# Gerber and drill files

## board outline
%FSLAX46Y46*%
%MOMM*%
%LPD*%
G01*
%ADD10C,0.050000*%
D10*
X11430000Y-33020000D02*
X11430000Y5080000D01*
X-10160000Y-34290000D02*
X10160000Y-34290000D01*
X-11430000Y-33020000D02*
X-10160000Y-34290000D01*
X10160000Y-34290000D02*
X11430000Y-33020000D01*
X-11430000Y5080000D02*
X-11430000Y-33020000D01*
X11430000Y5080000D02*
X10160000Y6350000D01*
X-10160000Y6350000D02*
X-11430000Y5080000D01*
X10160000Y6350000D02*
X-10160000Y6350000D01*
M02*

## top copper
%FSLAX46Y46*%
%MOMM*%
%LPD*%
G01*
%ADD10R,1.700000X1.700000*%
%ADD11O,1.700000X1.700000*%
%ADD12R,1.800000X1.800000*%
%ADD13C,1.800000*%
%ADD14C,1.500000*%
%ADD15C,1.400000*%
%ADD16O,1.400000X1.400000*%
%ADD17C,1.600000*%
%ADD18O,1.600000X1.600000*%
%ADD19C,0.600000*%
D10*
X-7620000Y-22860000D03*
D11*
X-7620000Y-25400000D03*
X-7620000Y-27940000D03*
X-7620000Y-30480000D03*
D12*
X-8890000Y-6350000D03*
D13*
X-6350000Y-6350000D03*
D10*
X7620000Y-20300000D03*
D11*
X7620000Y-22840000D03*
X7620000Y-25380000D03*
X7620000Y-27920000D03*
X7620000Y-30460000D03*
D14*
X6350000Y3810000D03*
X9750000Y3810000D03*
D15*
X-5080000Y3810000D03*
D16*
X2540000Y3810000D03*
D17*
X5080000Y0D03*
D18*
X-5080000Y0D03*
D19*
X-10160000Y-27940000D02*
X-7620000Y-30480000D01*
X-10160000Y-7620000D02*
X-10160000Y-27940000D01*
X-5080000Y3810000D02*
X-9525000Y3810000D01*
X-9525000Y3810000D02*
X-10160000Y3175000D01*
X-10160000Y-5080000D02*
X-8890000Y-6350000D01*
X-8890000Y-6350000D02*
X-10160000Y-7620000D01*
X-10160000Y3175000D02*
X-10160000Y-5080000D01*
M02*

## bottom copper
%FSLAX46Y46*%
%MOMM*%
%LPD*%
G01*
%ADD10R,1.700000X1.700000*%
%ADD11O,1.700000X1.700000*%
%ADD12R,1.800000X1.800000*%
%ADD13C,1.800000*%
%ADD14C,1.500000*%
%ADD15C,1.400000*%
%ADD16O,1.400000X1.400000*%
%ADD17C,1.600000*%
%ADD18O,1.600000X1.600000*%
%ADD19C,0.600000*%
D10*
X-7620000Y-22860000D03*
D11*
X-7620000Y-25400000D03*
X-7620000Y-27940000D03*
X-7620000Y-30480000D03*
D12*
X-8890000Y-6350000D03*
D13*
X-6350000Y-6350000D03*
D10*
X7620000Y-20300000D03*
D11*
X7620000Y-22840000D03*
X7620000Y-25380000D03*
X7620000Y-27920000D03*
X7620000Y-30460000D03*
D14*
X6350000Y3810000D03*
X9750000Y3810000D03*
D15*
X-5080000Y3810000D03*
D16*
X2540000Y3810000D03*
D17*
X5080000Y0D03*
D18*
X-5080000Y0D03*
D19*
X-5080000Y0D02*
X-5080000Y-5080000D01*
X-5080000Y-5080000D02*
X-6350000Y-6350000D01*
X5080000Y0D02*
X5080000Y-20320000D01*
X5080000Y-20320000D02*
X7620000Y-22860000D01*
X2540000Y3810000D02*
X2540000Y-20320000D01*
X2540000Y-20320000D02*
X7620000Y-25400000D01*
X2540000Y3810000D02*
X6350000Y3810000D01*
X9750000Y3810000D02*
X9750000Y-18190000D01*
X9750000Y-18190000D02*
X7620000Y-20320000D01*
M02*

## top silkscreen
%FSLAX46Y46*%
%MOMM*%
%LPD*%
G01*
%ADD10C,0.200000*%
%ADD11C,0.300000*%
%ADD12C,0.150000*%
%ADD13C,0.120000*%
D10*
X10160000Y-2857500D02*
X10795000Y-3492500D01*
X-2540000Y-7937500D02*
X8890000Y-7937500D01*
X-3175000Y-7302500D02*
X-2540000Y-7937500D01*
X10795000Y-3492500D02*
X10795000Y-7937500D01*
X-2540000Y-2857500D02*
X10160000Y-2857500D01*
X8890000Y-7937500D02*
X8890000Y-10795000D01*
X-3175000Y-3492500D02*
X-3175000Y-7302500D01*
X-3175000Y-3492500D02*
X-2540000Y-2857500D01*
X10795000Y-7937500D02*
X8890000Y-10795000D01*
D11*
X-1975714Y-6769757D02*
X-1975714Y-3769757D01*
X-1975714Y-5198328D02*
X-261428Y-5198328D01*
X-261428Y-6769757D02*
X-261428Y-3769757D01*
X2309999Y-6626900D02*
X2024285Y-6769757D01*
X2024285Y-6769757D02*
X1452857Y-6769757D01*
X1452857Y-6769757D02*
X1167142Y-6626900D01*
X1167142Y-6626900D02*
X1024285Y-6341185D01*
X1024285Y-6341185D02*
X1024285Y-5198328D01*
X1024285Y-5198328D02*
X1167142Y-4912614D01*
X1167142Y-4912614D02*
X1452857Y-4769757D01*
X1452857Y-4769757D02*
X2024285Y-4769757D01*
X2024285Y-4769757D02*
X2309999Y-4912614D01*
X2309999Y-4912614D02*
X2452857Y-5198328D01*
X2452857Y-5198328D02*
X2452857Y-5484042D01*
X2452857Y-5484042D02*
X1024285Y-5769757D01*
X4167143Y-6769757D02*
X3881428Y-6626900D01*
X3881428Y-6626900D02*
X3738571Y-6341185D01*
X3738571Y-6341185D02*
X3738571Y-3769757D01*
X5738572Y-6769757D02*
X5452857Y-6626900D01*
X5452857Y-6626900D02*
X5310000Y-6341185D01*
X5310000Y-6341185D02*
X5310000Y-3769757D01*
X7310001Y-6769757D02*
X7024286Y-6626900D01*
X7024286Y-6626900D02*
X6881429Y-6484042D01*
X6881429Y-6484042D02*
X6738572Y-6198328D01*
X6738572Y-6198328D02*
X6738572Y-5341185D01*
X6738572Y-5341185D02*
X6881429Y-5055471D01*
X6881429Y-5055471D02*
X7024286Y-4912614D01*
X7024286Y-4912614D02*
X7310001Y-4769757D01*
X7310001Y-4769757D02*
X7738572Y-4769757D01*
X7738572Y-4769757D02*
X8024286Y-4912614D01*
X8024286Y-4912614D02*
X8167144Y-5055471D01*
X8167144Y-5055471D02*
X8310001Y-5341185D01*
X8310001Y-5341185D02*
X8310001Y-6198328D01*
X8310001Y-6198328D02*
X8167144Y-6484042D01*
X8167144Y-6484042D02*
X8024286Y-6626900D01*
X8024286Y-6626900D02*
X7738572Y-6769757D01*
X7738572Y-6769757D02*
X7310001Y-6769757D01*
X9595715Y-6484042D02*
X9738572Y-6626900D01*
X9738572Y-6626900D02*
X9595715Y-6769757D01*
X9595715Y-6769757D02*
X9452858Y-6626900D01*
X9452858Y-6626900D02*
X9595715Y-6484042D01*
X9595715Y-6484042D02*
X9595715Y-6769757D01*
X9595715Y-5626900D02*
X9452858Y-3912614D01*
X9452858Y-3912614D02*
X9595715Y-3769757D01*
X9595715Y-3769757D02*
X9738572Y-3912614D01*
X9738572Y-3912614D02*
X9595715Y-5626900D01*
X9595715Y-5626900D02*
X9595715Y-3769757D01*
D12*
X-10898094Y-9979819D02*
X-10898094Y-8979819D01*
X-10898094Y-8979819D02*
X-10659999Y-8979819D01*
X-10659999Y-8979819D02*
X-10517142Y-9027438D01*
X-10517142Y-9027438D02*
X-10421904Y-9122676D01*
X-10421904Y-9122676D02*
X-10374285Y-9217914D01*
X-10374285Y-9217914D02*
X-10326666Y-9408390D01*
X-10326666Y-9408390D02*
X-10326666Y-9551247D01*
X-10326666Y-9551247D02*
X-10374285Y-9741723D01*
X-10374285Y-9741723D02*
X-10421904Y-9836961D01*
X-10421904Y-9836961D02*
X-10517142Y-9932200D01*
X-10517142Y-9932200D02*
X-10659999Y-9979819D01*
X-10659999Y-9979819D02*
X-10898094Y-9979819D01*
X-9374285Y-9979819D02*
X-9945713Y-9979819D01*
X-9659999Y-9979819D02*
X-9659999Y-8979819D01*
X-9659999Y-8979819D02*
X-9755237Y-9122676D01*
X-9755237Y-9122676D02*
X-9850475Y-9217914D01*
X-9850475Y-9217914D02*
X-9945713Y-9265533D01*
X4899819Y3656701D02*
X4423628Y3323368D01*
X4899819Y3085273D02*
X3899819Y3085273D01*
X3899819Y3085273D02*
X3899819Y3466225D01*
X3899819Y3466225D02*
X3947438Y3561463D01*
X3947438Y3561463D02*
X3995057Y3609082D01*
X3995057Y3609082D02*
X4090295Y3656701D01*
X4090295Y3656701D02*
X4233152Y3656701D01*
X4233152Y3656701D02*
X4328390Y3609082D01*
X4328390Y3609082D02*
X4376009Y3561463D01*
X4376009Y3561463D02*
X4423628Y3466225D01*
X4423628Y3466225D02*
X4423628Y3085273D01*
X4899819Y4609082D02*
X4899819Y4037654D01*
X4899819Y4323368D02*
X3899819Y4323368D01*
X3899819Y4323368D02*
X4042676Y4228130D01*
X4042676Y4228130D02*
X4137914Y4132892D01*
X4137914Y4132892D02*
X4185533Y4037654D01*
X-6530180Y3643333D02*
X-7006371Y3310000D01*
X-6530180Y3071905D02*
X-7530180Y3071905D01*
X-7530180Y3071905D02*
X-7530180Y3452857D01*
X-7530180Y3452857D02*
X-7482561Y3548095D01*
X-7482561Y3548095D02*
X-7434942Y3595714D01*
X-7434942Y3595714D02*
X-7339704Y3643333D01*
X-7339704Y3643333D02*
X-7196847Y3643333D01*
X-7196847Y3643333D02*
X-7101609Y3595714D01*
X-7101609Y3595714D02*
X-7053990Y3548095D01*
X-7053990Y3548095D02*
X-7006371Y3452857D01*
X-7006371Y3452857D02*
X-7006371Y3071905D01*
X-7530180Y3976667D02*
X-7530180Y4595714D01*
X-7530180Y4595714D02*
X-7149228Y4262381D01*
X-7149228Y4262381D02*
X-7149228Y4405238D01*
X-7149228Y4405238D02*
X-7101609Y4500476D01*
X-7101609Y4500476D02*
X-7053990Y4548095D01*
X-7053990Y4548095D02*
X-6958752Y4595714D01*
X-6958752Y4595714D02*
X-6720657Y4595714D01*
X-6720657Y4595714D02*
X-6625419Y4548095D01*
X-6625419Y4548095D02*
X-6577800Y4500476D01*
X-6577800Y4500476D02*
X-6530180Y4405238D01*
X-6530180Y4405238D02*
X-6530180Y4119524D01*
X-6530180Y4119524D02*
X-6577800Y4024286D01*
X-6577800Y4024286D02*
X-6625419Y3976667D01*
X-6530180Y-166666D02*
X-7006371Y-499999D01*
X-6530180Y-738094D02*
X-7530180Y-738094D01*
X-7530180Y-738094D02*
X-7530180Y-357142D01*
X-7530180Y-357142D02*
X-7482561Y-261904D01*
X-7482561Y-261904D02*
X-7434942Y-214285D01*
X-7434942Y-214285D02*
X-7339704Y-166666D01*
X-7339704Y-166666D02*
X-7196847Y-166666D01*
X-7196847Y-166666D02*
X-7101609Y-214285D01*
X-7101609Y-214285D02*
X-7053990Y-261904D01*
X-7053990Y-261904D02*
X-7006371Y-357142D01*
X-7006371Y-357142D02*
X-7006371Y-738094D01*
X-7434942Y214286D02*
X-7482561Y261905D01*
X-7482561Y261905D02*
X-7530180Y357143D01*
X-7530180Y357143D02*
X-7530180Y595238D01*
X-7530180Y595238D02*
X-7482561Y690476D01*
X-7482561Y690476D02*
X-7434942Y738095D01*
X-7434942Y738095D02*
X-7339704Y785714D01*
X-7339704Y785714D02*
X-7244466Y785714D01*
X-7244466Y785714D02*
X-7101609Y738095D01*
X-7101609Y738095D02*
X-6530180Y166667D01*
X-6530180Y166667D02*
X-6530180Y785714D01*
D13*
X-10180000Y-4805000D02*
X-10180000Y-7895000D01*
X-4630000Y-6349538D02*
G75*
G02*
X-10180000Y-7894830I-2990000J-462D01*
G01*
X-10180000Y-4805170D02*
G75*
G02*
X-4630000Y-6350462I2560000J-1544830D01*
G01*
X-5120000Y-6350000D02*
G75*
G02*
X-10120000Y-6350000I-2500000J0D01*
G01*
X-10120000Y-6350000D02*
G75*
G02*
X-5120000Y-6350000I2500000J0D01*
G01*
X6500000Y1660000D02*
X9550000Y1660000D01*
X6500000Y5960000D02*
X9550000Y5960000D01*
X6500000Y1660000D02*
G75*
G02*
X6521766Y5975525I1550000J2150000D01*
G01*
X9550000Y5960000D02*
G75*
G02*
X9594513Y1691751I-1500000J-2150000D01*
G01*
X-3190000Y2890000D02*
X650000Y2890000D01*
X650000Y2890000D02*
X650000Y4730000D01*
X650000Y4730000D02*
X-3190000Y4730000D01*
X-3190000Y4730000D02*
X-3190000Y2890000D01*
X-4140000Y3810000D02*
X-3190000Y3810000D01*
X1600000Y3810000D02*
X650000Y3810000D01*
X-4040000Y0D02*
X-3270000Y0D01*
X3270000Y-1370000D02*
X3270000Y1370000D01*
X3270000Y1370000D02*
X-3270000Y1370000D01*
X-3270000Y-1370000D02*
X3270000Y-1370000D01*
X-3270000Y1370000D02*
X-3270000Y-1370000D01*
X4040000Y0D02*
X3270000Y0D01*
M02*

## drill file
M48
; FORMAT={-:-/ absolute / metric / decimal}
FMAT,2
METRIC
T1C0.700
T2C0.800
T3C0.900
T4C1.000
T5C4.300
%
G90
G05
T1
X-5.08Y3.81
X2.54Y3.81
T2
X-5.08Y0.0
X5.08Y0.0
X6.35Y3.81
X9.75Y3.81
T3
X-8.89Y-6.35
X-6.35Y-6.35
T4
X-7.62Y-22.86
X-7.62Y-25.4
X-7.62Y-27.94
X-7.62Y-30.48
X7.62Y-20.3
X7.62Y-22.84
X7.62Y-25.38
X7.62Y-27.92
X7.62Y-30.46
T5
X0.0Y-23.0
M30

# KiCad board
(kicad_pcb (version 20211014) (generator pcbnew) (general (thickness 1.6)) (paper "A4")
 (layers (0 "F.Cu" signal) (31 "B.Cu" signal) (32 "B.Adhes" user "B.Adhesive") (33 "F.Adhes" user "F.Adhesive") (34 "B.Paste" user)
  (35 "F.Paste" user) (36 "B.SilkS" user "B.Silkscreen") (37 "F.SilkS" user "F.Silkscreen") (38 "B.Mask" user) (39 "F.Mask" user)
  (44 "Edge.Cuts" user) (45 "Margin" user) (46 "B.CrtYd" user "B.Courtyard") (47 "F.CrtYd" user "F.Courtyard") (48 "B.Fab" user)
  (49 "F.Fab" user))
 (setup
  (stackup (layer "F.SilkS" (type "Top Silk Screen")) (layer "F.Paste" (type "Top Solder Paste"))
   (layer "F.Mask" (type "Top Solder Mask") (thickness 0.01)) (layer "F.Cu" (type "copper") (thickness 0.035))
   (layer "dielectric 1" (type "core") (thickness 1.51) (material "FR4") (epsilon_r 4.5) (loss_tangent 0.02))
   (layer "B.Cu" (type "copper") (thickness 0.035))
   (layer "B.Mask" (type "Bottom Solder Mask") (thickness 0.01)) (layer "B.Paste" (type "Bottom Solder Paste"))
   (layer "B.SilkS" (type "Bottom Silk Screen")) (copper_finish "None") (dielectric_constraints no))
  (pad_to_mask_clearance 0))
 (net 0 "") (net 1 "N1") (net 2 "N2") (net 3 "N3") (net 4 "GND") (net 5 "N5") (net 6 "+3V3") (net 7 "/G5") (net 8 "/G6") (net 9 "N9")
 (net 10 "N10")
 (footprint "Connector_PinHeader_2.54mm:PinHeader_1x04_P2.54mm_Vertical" (layer "F.Cu") (at -7.62 22.86)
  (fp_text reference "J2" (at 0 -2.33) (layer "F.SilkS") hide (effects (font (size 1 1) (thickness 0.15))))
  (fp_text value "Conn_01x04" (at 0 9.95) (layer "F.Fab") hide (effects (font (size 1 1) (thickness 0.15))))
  (pad "1" thru_hole rect (at 0 0) (size 1.7 1.7) (drill 1) (layers *.Cu *.Mask) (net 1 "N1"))
  (pad "2" thru_hole oval (at 0 2.54) (size 1.7 1.7) (drill 1) (layers *.Cu *.Mask) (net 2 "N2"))
  (pad "3" thru_hole oval (at 0 5.08) (size 1.7 1.7) (drill 1) (layers *.Cu *.Mask) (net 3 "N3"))
  (pad "4" thru_hole oval (at 0 7.62) (size 1.7 1.7) (drill 1) (layers *.Cu *.Mask) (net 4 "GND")))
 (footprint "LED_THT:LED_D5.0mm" (layer "F.Cu") (at -8.89 6.35)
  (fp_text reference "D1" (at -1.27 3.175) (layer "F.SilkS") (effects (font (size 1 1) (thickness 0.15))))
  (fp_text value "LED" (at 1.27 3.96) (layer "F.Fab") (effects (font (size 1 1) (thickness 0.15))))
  (fp_line (start -1.29 -1.545) (end -1.29 1.545) (layer "F.SilkS") (width 0.12))
  (fp_arc (start 4.26 -0.000462) (mid 2.072002 2.880433) (end -1.29 1.54483) (layer "F.SilkS") (width 0.12))
  (fp_arc (start -1.29 -1.54483) (mid 2.072002 -2.880433) (end 4.26 0.000462) (layer "F.SilkS") (width 0.12))
  (fp_circle (center 1.27 0) (end 3.77 0) (layer "F.SilkS") (width 0.12) (fill none))
  (pad "1" thru_hole rect locked (at 0 0) (size 1.8 1.8) (drill 0.9) (layers *.Cu *.Mask) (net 4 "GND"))
  (pad "2" thru_hole circle locked (at 2.54 0) (size 1.8 1.8) (drill 0.9) (layers *.Cu *.Mask) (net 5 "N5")))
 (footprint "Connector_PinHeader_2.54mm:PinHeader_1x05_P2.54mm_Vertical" (layer "F.Cu") (at 7.62 20.3)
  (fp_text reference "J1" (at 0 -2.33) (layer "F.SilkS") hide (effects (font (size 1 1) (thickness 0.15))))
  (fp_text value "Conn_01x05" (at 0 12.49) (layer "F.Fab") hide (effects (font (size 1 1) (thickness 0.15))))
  (pad "1" thru_hole rect (at 0 0) (size 1.7 1.7) (drill 1) (layers *.Cu *.Mask) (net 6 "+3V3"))
  (pad "2" thru_hole oval (at 0 2.54) (size 1.7 1.7) (drill 1) (layers *.Cu *.Mask) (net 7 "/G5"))
  (pad "3" thru_hole oval (at 0 5.08) (size 1.7 1.7) (drill 1) (layers *.Cu *.Mask) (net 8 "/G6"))
  (pad "4" thru_hole oval (at 0 7.62) (size 1.7 1.7) (drill 1) (layers *.Cu *.Mask) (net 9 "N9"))
  (pad "5" thru_hole oval (at 0 10.16) (size 1.7 1.7) (drill 1) (layers *.Cu *.Mask) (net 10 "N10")))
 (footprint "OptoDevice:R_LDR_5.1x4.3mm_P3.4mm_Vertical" (layer "F.Cu") (at 6.35 -3.81)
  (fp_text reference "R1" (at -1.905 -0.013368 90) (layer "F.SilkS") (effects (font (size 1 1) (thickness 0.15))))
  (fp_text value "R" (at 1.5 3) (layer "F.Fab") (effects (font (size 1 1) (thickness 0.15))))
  (fp_line (start 0.15 2.15) (end 3.2 2.15) (layer "F.SilkS") (width 0.12))
  (fp_line (start 0.15 -2.15) (end 3.2 -2.15) (layer "F.SilkS") (width 0.12))
  (fp_arc (start 0.15 2.15) (mid -0.950438 -0.013368) (end 0.171766 -2.165525) (layer "F.SilkS") (width 0.12))
  (fp_arc (start 3.2 -2.15) (mid 4.321403 -0.027338) (end 3.244513 2.118249) (layer "F.SilkS") (width 0.12))
  (pad "1" thru_hole circle locked (at 0 0) (size 1.5 1.5) (drill 0.8) (layers *.Cu *.Mask) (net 8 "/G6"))
  (pad "2" thru_hole circle locked (at 3.4 0) (size 1.5 1.5) (drill 0.8) (layers *.Cu *.Mask) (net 6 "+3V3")))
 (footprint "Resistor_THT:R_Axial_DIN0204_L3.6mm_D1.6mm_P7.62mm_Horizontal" (layer "F.Cu") (at -5.08 -3.81)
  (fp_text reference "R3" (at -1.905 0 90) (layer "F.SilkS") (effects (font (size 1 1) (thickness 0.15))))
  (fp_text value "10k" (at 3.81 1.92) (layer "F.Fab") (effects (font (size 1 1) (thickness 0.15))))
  (fp_line (start 1.89 0.92) (end 5.73 0.92) (layer "F.SilkS") (width 0.12))
  (fp_line (start 5.73 0.92) (end 5.73 -0.92) (layer "F.SilkS") (width 0.12))
  (fp_line (start 5.73 -0.92) (end 1.89 -0.92) (layer "F.SilkS") (width 0.12))
  (fp_line (start 1.89 -0.92) (end 1.89 0.92) (layer "F.SilkS") (width 0.12))
  (fp_line (start 0.94 0) (end 1.89 0) (layer "F.SilkS") (width 0.12))
  (fp_line (start 6.68 0) (end 5.73 0) (layer "F.SilkS") (width 0.12))
  (pad "1" thru_hole circle locked (at 0 0) (size 1.4 1.4) (drill 0.7) (layers *.Cu *.Mask) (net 4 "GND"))
  (pad "2" thru_hole oval locked (at 7.62 0) (size 1.4 1.4) (drill 0.7) (layers *.Cu *.Mask) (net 8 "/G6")))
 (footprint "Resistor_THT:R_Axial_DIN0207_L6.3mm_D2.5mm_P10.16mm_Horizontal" (layer "F.Cu") (at 5.08 0 180)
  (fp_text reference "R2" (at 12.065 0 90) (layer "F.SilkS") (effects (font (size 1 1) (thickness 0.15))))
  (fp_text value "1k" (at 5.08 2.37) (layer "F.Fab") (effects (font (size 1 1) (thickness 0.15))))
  (fp_line (start 9.12 0) (end 8.35 0) (layer "F.SilkS") (width 0.12))
  (fp_line (start 1.81 -1.37) (end 1.81 1.37) (layer "F.SilkS") (width 0.12))
  (fp_line (start 1.81 1.37) (end 8.35 1.37) (layer "F.SilkS") (width 0.12))
  (fp_line (start 8.35 -1.37) (end 1.81 -1.37) (layer "F.SilkS") (width 0.12))
  (fp_line (start 8.35 1.37) (end 8.35 -1.37) (layer "F.SilkS") (width 0.12))
  (fp_line (start 1.04 0) (end 1.81 0) (layer "F.SilkS") (width 0.12))
  (pad "1" thru_hole circle locked (at 0 0 180) (size 1.6 1.6) (drill 0.8) (layers *.Cu *.Mask) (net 7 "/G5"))
  (pad "2" thru_hole oval locked (at 10.16 0 180) (size 1.6 1.6) (drill 0.8) (layers *.Cu *.Mask) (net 5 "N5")))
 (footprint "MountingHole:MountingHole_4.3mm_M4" (layer "F.Cu") (at 0 23)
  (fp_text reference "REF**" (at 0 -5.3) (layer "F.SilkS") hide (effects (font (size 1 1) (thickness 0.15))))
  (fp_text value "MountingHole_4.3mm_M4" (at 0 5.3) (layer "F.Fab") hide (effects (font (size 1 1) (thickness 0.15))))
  (pad "" np_thru_hole circle locked (at 0 0) (size 4.3 4.3) (drill 4.3) (layers *.Cu *.Mask)))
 (gr_line (start 10.16 2.8575) (end 10.795 3.4925) (layer "F.SilkS") (width 0.2))
 (gr_line (start -2.54 7.9375) (end 8.89 7.9375) (layer "F.SilkS") (width 0.2))
 (gr_line (start -3.175 7.3025) (end -2.54 7.9375) (layer "F.SilkS") (width 0.2))
 (gr_line (start 10.795 3.4925) (end 10.795 7.9375) (layer "F.SilkS") (width 0.2))
 (gr_line (start -2.54 2.8575) (end 10.16 2.8575) (layer "F.SilkS") (width 0.2))
 (gr_line (start 8.89 7.9375) (end 8.89 10.795) (layer "F.SilkS") (width 0.2))
 (gr_line (start -3.175 3.4925) (end -3.175 7.3025) (layer "F.SilkS") (width 0.2))
 (gr_line (start -3.175 3.4925) (end -2.54 2.8575) (layer "F.SilkS") (width 0.2))
 (gr_line (start 10.795 7.9375) (end 8.89 10.795) (layer "F.SilkS") (width 0.2))
 (gr_line (start 11.43 33.02) (end 11.43 -5.08) (layer "Edge.Cuts") (width 0.05))
 (gr_line (start -10.16 34.29) (end 10.16 34.29) (layer "Edge.Cuts") (width 0.05))
 (gr_line (start -11.43 33.02) (end -10.16 34.29) (layer "Edge.Cuts") (width 0.05))
 (gr_line (start 10.16 34.29) (end 11.43 33.02) (layer "Edge.Cuts") (width 0.05))
 (gr_line (start -11.43 -5.08) (end -11.43 33.02) (layer "Edge.Cuts") (width 0.05))
 (gr_line (start 11.43 -5.08) (end 10.16 -6.35) (layer "Edge.Cuts") (width 0.05))
 (gr_line (start -10.16 -6.35) (end -11.43 -5.08) (layer "Edge.Cuts") (width 0.05))
 (gr_line (start 10.16 -6.35) (end -10.16 -6.35) (layer "Edge.Cuts") (width 0.05))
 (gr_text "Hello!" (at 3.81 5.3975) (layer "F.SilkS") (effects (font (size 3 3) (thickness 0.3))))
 (segment (start -5.08 0) (end -5.08 5.08) (width 0.6) (layer "B.Cu") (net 5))
 (segment (start -5.08 5.08) (end -6.35 6.35) (width 0.6) (layer "B.Cu") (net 5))
 (segment (start 5.08 0) (end 5.08 20.32) (width 0.6) (layer "B.Cu") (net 7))
 (segment (start 5.08 20.32) (end 7.62 22.86) (width 0.6) (layer "B.Cu") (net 7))
 (segment (start -10.16 27.94) (end -7.62 30.48) (width 0.6) (layer "F.Cu") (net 4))
 (segment (start -10.16 7.62) (end -10.16 27.94) (width 0.6) (layer "F.Cu") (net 4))
 (segment (start -5.08 -3.81) (end -9.525 -3.81) (width 0.6) (layer "F.Cu") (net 4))
 (segment (start -9.525 -3.81) (end -10.16 -3.175) (width 0.6) (layer "F.Cu") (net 4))
 (segment (start -10.16 5.08) (end -8.89 6.35) (width 0.6) (layer "F.Cu") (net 4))
 (segment (start -8.89 6.35) (end -10.16 7.62) (width 0.6) (layer "F.Cu") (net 4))
 (segment (start -10.16 -3.175) (end -10.16 5.08) (width 0.6) (layer "F.Cu") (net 4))
 (segment (start 2.54 -3.81) (end 2.54 20.32) (width 0.6) (layer "B.Cu") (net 8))
 (segment (start 2.54 20.32) (end 7.62 25.4) (width 0.6) (layer "B.Cu") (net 8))
 (segment (start 2.54 -3.81) (end 6.35 -3.81) (width 0.6) (layer "B.Cu") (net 8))
 (segment (start 9.75 -3.81) (end 9.75 18.19) (width 0.6) (layer "B.Cu") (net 6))
 (segment (start 9.75 18.19) (end 7.62 20.32) (width 0.6) (layer "B.Cu") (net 6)))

